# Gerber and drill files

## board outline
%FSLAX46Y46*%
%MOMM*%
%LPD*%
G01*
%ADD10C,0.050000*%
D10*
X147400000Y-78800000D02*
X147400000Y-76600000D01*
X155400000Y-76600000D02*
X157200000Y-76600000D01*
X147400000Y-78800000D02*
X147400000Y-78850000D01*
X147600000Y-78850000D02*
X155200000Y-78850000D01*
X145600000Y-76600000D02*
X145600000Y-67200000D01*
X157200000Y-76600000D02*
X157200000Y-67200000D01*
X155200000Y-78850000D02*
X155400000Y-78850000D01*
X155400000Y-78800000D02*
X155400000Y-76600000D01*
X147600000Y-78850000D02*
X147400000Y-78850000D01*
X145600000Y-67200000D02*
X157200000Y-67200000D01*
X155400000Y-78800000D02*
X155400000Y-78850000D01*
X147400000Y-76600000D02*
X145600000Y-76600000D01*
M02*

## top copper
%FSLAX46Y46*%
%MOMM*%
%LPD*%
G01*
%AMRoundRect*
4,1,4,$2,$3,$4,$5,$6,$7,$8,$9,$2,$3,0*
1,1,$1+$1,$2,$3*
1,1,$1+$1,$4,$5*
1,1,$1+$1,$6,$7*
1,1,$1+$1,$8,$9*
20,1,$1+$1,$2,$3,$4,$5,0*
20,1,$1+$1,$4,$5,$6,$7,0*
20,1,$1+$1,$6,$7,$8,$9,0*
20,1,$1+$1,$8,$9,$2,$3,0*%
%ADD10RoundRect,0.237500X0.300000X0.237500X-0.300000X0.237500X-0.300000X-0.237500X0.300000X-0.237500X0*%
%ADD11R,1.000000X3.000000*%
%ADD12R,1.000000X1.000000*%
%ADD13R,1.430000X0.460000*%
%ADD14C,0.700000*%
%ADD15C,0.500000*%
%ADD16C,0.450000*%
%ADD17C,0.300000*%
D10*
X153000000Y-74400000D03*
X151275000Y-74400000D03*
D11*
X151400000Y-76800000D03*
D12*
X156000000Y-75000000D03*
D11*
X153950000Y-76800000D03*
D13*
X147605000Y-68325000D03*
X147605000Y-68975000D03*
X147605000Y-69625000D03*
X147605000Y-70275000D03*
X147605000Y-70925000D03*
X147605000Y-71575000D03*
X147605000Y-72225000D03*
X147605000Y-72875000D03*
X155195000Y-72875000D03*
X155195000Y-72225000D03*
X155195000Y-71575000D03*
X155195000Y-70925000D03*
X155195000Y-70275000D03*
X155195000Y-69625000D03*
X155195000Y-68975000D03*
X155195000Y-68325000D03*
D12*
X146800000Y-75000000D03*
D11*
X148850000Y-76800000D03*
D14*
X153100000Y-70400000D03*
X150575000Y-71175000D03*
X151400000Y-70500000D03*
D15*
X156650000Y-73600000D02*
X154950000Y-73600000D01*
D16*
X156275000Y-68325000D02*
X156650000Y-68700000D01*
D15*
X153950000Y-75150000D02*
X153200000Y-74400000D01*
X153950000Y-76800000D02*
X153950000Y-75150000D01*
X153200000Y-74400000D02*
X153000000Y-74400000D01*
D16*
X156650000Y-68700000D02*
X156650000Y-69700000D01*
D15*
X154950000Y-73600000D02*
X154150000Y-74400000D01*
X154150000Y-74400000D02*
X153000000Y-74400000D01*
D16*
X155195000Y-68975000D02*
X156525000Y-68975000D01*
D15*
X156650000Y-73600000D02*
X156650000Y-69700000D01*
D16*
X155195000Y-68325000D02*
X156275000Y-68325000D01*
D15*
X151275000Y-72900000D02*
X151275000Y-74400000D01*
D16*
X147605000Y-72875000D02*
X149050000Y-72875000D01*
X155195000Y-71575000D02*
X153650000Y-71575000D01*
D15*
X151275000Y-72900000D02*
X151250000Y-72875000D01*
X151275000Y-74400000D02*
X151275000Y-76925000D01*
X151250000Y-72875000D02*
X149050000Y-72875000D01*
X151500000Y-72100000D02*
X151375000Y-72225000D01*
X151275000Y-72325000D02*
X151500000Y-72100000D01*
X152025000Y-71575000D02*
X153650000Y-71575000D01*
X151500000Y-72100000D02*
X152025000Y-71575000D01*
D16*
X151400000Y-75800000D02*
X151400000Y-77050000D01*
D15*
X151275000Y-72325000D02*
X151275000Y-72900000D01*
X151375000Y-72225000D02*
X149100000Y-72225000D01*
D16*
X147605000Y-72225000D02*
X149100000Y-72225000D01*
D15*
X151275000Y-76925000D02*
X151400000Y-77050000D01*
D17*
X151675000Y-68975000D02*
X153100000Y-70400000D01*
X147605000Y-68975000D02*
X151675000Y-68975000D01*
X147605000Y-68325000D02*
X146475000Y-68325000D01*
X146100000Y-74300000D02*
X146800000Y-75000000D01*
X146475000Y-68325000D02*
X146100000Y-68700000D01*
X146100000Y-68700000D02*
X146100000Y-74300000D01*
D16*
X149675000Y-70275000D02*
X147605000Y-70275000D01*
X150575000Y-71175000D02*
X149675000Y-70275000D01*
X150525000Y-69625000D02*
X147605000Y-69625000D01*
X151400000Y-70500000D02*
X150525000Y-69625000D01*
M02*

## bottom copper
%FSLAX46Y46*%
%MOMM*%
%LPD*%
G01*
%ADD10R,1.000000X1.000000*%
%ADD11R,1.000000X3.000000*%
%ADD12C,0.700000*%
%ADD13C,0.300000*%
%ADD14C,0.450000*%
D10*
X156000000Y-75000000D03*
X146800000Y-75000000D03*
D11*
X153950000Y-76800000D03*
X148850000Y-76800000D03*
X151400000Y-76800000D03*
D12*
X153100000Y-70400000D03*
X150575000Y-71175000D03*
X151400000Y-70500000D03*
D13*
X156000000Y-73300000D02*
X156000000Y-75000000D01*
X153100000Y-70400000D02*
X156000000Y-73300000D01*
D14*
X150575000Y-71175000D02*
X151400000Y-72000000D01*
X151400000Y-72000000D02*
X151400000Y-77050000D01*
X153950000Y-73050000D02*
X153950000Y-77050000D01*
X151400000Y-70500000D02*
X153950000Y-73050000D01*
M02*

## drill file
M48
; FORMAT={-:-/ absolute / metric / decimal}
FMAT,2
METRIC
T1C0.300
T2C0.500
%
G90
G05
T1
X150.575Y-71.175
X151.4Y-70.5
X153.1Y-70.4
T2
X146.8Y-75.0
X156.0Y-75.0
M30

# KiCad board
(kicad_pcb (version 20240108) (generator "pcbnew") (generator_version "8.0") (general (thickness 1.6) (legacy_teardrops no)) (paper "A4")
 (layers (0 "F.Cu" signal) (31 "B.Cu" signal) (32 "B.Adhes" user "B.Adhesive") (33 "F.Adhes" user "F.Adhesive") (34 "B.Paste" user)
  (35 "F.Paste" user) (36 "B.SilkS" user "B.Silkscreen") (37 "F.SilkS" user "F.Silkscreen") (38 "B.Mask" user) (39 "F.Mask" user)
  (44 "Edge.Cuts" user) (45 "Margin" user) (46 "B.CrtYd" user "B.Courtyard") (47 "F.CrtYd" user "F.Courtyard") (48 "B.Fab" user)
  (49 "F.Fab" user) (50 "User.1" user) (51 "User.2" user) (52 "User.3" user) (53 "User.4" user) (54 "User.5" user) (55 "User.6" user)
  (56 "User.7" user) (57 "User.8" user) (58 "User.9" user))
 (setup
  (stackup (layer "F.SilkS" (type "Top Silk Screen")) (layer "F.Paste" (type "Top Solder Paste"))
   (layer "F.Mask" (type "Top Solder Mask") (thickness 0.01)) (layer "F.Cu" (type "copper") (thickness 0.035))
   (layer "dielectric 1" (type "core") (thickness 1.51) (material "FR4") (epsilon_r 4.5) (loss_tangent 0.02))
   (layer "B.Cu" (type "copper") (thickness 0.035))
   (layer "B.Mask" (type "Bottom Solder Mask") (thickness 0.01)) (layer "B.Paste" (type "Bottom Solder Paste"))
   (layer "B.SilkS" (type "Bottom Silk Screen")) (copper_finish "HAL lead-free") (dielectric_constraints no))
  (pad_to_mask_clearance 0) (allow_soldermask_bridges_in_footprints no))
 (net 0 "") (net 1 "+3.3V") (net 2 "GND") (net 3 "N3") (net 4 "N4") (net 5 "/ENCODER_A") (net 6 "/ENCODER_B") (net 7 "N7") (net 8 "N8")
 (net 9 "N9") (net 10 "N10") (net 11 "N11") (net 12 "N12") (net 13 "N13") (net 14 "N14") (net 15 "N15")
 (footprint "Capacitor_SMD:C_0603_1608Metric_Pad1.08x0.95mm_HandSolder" (layer "F.Cu") (at 152.1375 74.4 180)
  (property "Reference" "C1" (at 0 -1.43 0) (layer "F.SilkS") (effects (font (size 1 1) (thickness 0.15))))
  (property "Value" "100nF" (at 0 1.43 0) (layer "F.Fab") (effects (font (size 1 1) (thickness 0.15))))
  (pad "1" smd roundrect (at -0.8625 0 180) (size 1.075 0.95) (layers "F.Cu" "F.Paste" "F.Mask") (roundrect_rratio 0.25) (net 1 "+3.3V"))
  (pad "2" smd roundrect (at 0.8625 0 180) (size 1.075 0.95) (layers "F.Cu" "F.Paste" "F.Mask") (roundrect_rratio 0.25) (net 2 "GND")))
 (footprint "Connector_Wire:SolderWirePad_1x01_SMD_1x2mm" (layer "F.Cu") (at 151.4 76.8)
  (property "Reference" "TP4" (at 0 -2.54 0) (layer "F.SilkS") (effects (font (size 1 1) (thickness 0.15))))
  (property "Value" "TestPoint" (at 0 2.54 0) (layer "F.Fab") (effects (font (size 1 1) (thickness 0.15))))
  (pad "1" smd rect (at 0 0) (size 1 3) (layers "F.Cu" "F.Paste" "F.Mask") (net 2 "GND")))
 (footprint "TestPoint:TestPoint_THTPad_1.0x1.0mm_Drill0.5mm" (layer "F.Cu") (at 156 75)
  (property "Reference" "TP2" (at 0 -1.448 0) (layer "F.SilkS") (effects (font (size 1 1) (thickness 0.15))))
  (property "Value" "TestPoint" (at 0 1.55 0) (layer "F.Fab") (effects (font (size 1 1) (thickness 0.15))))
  (pad "1" thru_hole rect (at 0 0) (size 1 1) (drill 0.5) (layers "*.Cu" "*.Mask") (remove_unused_layers no) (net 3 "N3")))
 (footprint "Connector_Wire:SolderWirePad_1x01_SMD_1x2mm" (layer "F.Cu") (at 153.95 76.8 180)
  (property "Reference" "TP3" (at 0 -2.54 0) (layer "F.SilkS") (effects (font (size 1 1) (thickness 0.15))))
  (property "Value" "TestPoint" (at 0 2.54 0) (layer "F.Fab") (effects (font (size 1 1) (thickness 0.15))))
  (pad "1" smd rect (at 0 0 180) (size 1 3) (layers "F.Cu" "F.Paste" "F.Mask") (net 1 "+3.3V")))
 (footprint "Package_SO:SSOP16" (layer "F.Cu") (at 151.4 70.6 -90)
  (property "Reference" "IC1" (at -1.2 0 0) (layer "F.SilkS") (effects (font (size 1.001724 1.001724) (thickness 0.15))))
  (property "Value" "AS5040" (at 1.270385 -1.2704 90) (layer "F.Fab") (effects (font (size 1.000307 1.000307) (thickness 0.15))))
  (pad "1" smd rect (at -2.275 3.795 270) (size 0.46 1.43) (layers "F.Cu" "F.Paste" "F.Mask") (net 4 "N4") (solder_mask_margin 0.102))
  (pad "2" smd rect (at -1.625 3.795 270) (size 0.46 1.43) (layers "F.Cu" "F.Paste" "F.Mask") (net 3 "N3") (solder_mask_margin 0.102))
  (pad "3" smd rect (at -0.975 3.795 270) (size 0.46 1.43) (layers "F.Cu" "F.Paste" "F.Mask") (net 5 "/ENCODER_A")
   (solder_mask_margin 0.102))
  (pad "4" smd rect (at -0.325 3.795 270) (size 0.46 1.43) (layers "F.Cu" "F.Paste" "F.Mask") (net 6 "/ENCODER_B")
   (solder_mask_margin 0.102))
  (pad "5" smd rect (at 0.325 3.795 270) (size 0.46 1.43) (layers "F.Cu" "F.Paste" "F.Mask") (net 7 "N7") (solder_mask_margin 0.102))
  (pad "6" smd rect (at 0.975 3.795 270) (size 0.46 1.43) (layers "F.Cu" "F.Paste" "F.Mask") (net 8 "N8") (solder_mask_margin 0.102))
  (pad "7" smd rect (at 1.625 3.795 270) (size 0.46 1.43) (layers "F.Cu" "F.Paste" "F.Mask") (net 2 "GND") (solder_mask_margin 0.102))
  (pad "8" smd rect (at 2.275 3.795 270) (size 0.46 1.43) (layers "F.Cu" "F.Paste" "F.Mask") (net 2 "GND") (solder_mask_margin 0.102))
  (pad "9" smd rect (at 2.275 -3.795 270) (size 0.46 1.43) (layers "F.Cu" "F.Paste" "F.Mask") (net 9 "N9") (solder_mask_margin 0.102))
  (pad "10" smd rect (at 1.625 -3.795 270) (size 0.46 1.43) (layers "F.Cu" "F.Paste" "F.Mask") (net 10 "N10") (solder_mask_margin 0.102))
  (pad "11" smd rect (at 0.975 -3.795 270) (size 0.46 1.43) (layers "F.Cu" "F.Paste" "F.Mask") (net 2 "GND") (solder_mask_margin 0.102))
  (pad "12" smd rect (at 0.325 -3.795 270) (size 0.46 1.43) (layers "F.Cu" "F.Paste" "F.Mask") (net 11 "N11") (solder_mask_margin 0.102))
  (pad "13" smd rect (at -0.325 -3.795 270) (size 0.46 1.43) (layers "F.Cu" "F.Paste" "F.Mask") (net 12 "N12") (solder_mask_margin 0.102))
  (pad "14" smd rect (at -0.975 -3.795 270) (size 0.46 1.43) (layers "F.Cu" "F.Paste" "F.Mask") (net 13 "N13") (solder_mask_margin 0.102))
  (pad "15" smd rect (at -1.625 -3.795 270) (size 0.46 1.43) (layers "F.Cu" "F.Paste" "F.Mask") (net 1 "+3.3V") (solder_mask_margin 0.102))
  (pad "16" smd rect (at -2.275 -3.795 270) (size 0.46 1.43) (layers "F.Cu" "F.Paste" "F.Mask") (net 1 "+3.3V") (solder_mask_margin 0.102)))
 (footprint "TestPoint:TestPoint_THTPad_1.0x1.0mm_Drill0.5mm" (layer "F.Cu") (at 146.8 75)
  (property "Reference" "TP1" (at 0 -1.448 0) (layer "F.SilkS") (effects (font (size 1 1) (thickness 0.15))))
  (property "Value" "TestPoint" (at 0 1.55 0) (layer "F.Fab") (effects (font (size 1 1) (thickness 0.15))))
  (pad "1" thru_hole rect (at 0 0) (size 1 1) (drill 0.5) (layers "*.Cu" "*.Mask") (remove_unused_layers no) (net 4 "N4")))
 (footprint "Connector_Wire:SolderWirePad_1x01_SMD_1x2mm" (layer "F.Cu") (at 148.85 76.8)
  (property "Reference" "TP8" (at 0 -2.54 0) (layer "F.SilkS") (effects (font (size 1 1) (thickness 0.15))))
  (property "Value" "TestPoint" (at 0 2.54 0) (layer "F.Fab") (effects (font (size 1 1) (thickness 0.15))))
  (pad "1" smd rect (at 0 0) (size 1 3) (layers "F.Cu" "F.Paste" "F.Mask") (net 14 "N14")))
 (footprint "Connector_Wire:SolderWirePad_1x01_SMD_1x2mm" (layer "B.Cu") (at 153.95 76.8 180)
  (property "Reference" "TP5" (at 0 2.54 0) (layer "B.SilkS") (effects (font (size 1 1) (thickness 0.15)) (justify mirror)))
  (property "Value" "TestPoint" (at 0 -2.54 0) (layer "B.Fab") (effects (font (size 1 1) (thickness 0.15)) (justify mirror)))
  (pad "1" smd rect (at 0 0 180) (size 1 3) (layers "B.Cu" "B.Paste" "B.Mask") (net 5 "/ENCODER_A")))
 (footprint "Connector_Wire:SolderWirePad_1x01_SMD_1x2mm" (layer "B.Cu") (at 148.85 76.8 180)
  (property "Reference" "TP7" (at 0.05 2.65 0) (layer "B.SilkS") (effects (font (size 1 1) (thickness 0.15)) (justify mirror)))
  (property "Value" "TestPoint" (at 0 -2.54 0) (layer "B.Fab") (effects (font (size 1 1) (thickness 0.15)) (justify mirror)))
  (pad "1" smd rect (at 0 0 180) (size 1 3) (layers "B.Cu" "B.Paste" "B.Mask") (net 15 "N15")))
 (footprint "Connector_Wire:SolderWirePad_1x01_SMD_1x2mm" (layer "B.Cu") (at 151.4 76.8 180)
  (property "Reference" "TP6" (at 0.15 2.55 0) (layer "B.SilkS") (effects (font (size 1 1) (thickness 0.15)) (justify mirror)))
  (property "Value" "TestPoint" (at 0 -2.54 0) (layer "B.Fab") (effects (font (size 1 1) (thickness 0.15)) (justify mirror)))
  (pad "1" smd rect (at 0 0 180) (size 1 3) (layers "B.Cu" "B.Paste" "B.Mask") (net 6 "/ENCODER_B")))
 (gr_line (start 147.4 78.8) (end 147.4 76.6) (stroke (width 0.05) (type default)) (layer "Edge.Cuts"))
 (gr_line (start 155.4 76.6) (end 157.2 76.6) (stroke (width 0.05) (type default)) (layer "Edge.Cuts"))
 (gr_line (start 147.4 78.8) (end 147.4 78.85) (stroke (width 0.05) (type default)) (layer "Edge.Cuts"))
 (gr_line (start 147.6 78.85) (end 155.2 78.85) (stroke (width 0.05) (type default)) (layer "Edge.Cuts"))
 (gr_line (start 145.6 76.6) (end 145.6 67.2) (stroke (width 0.05) (type default)) (layer "Edge.Cuts"))
 (gr_line (start 157.2 76.6) (end 157.2 67.2) (stroke (width 0.05) (type default)) (layer "Edge.Cuts"))
 (gr_line (start 155.2 78.85) (end 155.4 78.85) (stroke (width 0.05) (type default)) (layer "Edge.Cuts"))
 (gr_line (start 155.4 78.8) (end 155.4 76.6) (stroke (width 0.05) (type default)) (layer "Edge.Cuts"))
 (gr_line (start 147.6 78.85) (end 147.4 78.85) (stroke (width 0.05) (type default)) (layer "Edge.Cuts"))
 (gr_line (start 145.6 67.2) (end 157.2 67.2) (stroke (width 0.05) (type default)) (layer "Edge.Cuts"))
 (gr_line (start 155.4 78.8) (end 155.4 78.85) (stroke (width 0.05) (type default)) (layer "Edge.Cuts"))
 (gr_line (start 147.4 76.6) (end 145.6 76.6) (stroke (width 0.05) (type default)) (layer "Edge.Cuts"))
 (segment (start 156.65 73.6) (end 154.95 73.6) (width 0.5) (layer "F.Cu") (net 1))
 (segment (start 156.275 68.325) (end 156.65 68.7) (width 0.45) (layer "F.Cu") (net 1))
 (segment (start 153.95 75.15) (end 153.2 74.4) (width 0.5) (layer "F.Cu") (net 1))
 (segment (start 153.95 76.8) (end 153.95 75.15) (width 0.5) (layer "F.Cu") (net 1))
 (segment (start 153.2 74.4) (end 153 74.4) (width 0.5) (layer "F.Cu") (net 1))
 (segment (start 156.65 68.7) (end 156.65 69.7) (width 0.45) (layer "F.Cu") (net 1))
 (segment (start 154.95 73.6) (end 154.15 74.4) (width 0.5) (layer "F.Cu") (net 1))
 (segment (start 154.15 74.4) (end 153 74.4) (width 0.5) (layer "F.Cu") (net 1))
 (segment (start 155.195 68.975) (end 156.525 68.975) (width 0.45) (layer "F.Cu") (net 1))
 (segment (start 156.65 73.6) (end 156.65 69.7) (width 0.5) (layer "F.Cu") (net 1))
 (segment (start 155.195 68.325) (end 156.275 68.325) (width 0.45) (layer "F.Cu") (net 1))
 (segment (start 151.275 72.9) (end 151.275 74.4) (width 0.5) (layer "F.Cu") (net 2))
 (segment (start 147.605 72.875) (end 149.05 72.875) (width 0.45) (layer "F.Cu") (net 2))
 (segment (start 155.195 71.575) (end 153.65 71.575) (width 0.45) (layer "F.Cu") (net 2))
 (segment (start 151.275 72.9) (end 151.25 72.875) (width 0.5) (layer "F.Cu") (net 2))
 (segment (start 151.275 74.4) (end 151.275 76.925) (width 0.5) (layer "F.Cu") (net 2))
 (segment (start 151.25 72.875) (end 149.05 72.875) (width 0.5) (layer "F.Cu") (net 2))
 (segment (start 151.5 72.1) (end 151.375 72.225) (width 0.5) (layer "F.Cu") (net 2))
 (segment (start 151.275 72.325) (end 151.5 72.1) (width 0.5) (layer "F.Cu") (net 2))
 (segment (start 152.025 71.575) (end 153.65 71.575) (width 0.5) (layer "F.Cu") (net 2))
 (segment (start 151.5 72.1) (end 152.025 71.575) (width 0.5) (layer "F.Cu") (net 2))
 (segment (start 151.4 75.8) (end 151.4 77.05) (width 0.45) (layer "F.Cu") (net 2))
 (segment (start 151.275 72.325) (end 151.275 72.9) (width 0.5) (layer "F.Cu") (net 2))
 (segment (start 151.375 72.225) (end 149.1 72.225) (width 0.5) (layer "F.Cu") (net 2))
 (segment (start 147.605 72.225) (end 149.1 72.225) (width 0.45) (layer "F.Cu") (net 2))
 (segment (start 151.275 76.925) (end 151.4 77.05) (width 0.5) (layer "F.Cu") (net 2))
 (segment (start 151.675 68.975) (end 153.1 70.4) (width 0.3) (layer "F.Cu") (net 3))
 (segment (start 147.605 68.975) (end 151.675 68.975) (width 0.3) (layer "F.Cu") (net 3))
 (via (at 153.1 70.4) (size 0.7) (drill 0.3) (layers "F.Cu" "B.Cu") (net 3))
 (segment (start 156 73.3) (end 156 75) (width 0.3) (layer "B.Cu") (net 3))
 (segment (start 153.1 70.4) (end 156 73.3) (width 0.3) (layer "B.Cu") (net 3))
 (segment (start 147.605 68.325) (end 146.475 68.325) (width 0.3) (layer "F.Cu") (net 4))
 (segment (start 146.1 74.3) (end 146.8 75) (width 0.3) (layer "F.Cu") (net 4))
 (segment (start 146.475 68.325) (end 146.1 68.7) (width 0.3) (layer "F.Cu") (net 4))
 (segment (start 146.1 68.7) (end 146.1 74.3) (width 0.3) (layer "F.Cu") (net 4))
 (segment (start 149.675 70.275) (end 147.605 70.275) (width 0.45) (layer "F.Cu") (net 6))
 (segment (start 150.575 71.175) (end 149.675 70.275) (width 0.45) (layer "F.Cu") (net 6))
 (via (at 150.575 71.175) (size 0.7) (drill 0.3) (layers "F.Cu" "B.Cu") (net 6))
 (segment (start 150.575 71.175) (end 151.4 72) (width 0.45) (layer "B.Cu") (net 6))
 (segment (start 151.4 72) (end 151.4 77.05) (width 0.45) (layer "B.Cu") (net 6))
 (segment (start 150.525 69.625) (end 147.605 69.625) (width 0.45) (layer "F.Cu") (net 5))
 (segment (start 151.4 70.5) (end 150.525 69.625) (width 0.45) (layer "F.Cu") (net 5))
 (via (at 151.4 70.5) (size 0.7) (drill 0.3) (layers "F.Cu" "B.Cu") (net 5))
 (segment (start 153.95 73.05) (end 153.95 77.05) (width 0.45) (layer "B.Cu") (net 5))
 (segment (start 151.4 70.5) (end 153.95 73.05) (width 0.45) (layer "B.Cu") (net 5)))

